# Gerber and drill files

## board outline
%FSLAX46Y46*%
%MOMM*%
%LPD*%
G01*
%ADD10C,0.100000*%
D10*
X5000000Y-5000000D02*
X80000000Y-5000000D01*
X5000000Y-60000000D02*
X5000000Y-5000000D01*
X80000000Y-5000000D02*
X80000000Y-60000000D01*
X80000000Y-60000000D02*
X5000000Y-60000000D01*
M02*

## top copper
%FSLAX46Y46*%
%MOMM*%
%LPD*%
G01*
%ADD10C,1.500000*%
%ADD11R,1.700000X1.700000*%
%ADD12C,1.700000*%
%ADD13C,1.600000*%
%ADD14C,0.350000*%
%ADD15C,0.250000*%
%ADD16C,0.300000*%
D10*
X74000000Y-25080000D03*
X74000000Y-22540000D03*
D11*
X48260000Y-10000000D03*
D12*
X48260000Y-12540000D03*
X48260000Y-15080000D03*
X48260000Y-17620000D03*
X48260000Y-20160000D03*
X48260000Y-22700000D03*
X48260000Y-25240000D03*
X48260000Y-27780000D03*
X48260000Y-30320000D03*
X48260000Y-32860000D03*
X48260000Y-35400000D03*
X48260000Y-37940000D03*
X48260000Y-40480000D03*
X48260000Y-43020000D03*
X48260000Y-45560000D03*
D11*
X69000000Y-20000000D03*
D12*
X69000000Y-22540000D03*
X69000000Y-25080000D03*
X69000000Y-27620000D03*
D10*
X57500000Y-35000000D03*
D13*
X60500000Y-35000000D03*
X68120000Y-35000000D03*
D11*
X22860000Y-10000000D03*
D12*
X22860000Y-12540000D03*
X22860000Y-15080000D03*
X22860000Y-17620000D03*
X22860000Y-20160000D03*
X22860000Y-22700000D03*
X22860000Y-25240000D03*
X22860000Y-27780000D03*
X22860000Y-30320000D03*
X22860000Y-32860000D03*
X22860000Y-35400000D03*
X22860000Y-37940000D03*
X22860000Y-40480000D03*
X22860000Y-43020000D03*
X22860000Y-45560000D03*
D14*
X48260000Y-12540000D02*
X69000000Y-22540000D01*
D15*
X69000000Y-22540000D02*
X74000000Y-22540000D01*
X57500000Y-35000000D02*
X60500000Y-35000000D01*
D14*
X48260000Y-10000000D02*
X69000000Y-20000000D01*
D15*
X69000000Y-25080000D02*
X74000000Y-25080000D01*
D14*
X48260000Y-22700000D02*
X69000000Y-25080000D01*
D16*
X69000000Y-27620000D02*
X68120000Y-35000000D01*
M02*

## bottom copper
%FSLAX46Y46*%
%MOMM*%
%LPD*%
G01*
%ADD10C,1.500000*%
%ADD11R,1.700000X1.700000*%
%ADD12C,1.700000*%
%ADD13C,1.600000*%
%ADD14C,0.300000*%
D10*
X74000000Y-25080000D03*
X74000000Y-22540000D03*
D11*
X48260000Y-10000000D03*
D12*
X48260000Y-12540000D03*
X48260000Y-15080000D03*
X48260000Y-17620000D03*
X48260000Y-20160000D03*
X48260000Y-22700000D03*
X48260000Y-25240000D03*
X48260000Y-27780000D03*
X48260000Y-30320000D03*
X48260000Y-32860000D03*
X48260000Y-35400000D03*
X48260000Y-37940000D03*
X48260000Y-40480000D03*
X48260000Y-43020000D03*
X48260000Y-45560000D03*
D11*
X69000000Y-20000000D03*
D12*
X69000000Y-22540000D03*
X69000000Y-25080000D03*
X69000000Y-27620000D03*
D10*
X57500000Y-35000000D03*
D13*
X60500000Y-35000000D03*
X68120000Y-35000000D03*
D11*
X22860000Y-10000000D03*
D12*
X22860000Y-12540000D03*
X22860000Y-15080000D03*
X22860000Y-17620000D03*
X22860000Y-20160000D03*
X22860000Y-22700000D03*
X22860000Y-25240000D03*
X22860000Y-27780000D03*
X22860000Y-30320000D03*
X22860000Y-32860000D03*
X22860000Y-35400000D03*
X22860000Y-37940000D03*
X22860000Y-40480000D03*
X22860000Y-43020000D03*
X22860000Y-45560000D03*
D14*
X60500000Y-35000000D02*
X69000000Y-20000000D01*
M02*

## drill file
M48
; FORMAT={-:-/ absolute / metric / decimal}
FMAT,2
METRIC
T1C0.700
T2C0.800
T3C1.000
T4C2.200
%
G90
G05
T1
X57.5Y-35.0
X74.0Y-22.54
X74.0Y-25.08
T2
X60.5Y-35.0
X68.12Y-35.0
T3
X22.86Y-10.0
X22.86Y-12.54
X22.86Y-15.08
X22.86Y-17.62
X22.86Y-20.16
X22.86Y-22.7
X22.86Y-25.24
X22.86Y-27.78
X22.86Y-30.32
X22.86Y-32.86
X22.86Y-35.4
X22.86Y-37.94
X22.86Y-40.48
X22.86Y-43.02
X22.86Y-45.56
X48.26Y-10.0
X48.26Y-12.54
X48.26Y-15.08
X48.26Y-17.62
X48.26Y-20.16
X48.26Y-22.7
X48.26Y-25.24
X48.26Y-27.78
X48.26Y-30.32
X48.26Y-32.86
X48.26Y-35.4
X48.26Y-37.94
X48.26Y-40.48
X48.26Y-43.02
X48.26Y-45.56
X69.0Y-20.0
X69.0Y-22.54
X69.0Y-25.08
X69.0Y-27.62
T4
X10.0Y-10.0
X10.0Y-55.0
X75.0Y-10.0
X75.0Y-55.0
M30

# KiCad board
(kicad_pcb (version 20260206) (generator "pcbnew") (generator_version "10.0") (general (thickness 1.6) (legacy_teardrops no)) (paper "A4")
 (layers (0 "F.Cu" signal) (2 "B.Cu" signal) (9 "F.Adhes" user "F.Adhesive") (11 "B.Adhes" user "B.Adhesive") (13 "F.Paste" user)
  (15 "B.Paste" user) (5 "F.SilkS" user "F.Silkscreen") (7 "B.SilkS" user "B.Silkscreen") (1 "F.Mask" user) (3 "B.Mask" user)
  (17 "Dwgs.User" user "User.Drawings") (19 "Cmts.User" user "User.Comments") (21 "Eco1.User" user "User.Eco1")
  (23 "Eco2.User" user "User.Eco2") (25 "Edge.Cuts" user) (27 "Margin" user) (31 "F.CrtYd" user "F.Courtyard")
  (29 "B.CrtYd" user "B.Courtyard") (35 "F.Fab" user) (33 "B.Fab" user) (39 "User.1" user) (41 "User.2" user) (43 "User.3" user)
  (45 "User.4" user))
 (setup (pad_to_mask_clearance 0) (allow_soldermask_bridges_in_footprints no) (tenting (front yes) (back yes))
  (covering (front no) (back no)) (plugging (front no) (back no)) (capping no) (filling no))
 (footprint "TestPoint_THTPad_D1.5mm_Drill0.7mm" (layer "F.Cu") (at 74 25.08)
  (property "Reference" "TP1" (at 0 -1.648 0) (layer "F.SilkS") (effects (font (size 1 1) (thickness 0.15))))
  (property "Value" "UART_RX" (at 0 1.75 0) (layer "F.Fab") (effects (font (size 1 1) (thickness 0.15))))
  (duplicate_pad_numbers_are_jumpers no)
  (pad "1" thru_hole circle (at 0 0) (size 1.5 1.5) (drill 0.7) (layers "*.Cu" "*.Mask") (remove_unused_layers no) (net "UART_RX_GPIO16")))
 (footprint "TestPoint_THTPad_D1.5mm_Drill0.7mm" (layer "F.Cu") (at 74 22.54)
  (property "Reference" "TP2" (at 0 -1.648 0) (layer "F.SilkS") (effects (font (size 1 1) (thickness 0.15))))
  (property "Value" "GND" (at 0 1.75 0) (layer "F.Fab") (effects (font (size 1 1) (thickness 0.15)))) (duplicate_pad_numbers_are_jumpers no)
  (pad "1" thru_hole circle (at 0 0) (size 1.5 1.5) (drill 0.7) (layers "*.Cu" "*.Mask") (remove_unused_layers no) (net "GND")))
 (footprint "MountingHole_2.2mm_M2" (layer "F.Cu") (at 10 55)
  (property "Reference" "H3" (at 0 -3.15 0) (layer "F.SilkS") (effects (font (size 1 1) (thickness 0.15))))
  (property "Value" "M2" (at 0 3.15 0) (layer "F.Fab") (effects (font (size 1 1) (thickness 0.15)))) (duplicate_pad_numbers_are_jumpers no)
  (pad "" np_thru_hole circle (at 0 0) (size 2.2 2.2) (drill 2.2) (layers "*.Cu" "*.Mask")))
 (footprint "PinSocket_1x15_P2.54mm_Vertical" (layer "F.Cu") (at 48.26 10)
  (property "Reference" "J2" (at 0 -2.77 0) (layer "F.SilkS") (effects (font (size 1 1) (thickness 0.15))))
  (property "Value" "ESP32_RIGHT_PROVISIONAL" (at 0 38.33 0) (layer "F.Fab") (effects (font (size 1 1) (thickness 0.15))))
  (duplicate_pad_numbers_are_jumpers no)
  (pad "1" thru_hole rect (at 0 0) (size 1.7 1.7) (drill 1) (layers "*.Cu" "*.Mask") (remove_unused_layers no) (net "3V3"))
  (pad "2" thru_hole circle (at 0 2.54) (size 1.7 1.7) (drill 1) (layers "*.Cu" "*.Mask") (remove_unused_layers no) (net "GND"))
  (pad "3" thru_hole circle (at 0 5.08) (size 1.7 1.7) (drill 1) (layers "*.Cu" "*.Mask") (remove_unused_layers no))
  (pad "4" thru_hole circle (at 0 7.62) (size 1.7 1.7) (drill 1) (layers "*.Cu" "*.Mask") (remove_unused_layers no))
  (pad "5" thru_hole circle (at 0 10.16) (size 1.7 1.7) (drill 1) (layers "*.Cu" "*.Mask") (remove_unused_layers no))
  (pad "6" thru_hole circle (at 0 12.7) (size 1.7 1.7) (drill 1) (layers "*.Cu" "*.Mask") (remove_unused_layers no) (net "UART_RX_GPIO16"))
  (pad "7" thru_hole circle (at 0 15.24) (size 1.7 1.7) (drill 1) (layers "*.Cu" "*.Mask") (remove_unused_layers no))
  (pad "8" thru_hole circle (at 0 17.78) (size 1.7 1.7) (drill 1) (layers "*.Cu" "*.Mask") (remove_unused_layers no))
  (pad "9" thru_hole circle (at 0 20.32) (size 1.7 1.7) (drill 1) (layers "*.Cu" "*.Mask") (remove_unused_layers no))
  (pad "10" thru_hole circle (at 0 22.86) (size 1.7 1.7) (drill 1) (layers "*.Cu" "*.Mask") (remove_unused_layers no))
  (pad "11" thru_hole circle (at 0 25.4) (size 1.7 1.7) (drill 1) (layers "*.Cu" "*.Mask") (remove_unused_layers no))
  (pad "12" thru_hole circle (at 0 27.94) (size 1.7 1.7) (drill 1) (layers "*.Cu" "*.Mask") (remove_unused_layers no))
  (pad "13" thru_hole circle (at 0 30.48) (size 1.7 1.7) (drill 1) (layers "*.Cu" "*.Mask") (remove_unused_layers no))
  (pad "14" thru_hole circle (at 0 33.02) (size 1.7 1.7) (drill 1) (layers "*.Cu" "*.Mask") (remove_unused_layers no))
  (pad "15" thru_hole circle (at 0 35.56) (size 1.7 1.7) (drill 1) (layers "*.Cu" "*.Mask") (remove_unused_layers no)))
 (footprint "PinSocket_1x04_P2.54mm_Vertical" (layer "F.Cu") (at 69 20)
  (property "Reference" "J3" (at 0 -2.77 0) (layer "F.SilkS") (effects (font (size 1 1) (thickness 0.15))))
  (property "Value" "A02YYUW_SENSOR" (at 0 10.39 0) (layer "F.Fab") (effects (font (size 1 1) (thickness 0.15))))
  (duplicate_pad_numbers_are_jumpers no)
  (pad "1" thru_hole rect (at 0 0) (size 1.7 1.7) (drill 1) (layers "*.Cu" "*.Mask") (remove_unused_layers no) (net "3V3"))
  (pad "2" thru_hole circle (at 0 2.54) (size 1.7 1.7) (drill 1) (layers "*.Cu" "*.Mask") (remove_unused_layers no) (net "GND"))
  (pad "3" thru_hole circle (at 0 5.08) (size 1.7 1.7) (drill 1) (layers "*.Cu" "*.Mask") (remove_unused_layers no) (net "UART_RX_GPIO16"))
  (pad "4" thru_hole circle (at 0 7.62) (size 1.7 1.7) (drill 1) (layers "*.Cu" "*.Mask") (remove_unused_layers no) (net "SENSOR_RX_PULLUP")))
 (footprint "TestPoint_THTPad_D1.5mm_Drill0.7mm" (layer "F.Cu") (at 57.5 35)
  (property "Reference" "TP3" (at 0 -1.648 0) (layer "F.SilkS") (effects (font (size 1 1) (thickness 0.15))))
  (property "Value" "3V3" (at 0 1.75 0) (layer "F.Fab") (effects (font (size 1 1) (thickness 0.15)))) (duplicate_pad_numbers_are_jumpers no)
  (pad "1" thru_hole circle (at 0 0) (size 1.5 1.5) (drill 0.7) (layers "*.Cu" "*.Mask") (remove_unused_layers no) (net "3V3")))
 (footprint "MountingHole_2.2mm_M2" (layer "F.Cu") (at 10 10)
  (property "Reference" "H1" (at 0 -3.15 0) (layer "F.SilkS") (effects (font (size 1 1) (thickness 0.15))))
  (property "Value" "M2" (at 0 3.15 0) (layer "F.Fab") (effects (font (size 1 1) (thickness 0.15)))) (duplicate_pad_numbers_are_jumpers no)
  (pad "" np_thru_hole circle (at 0 0) (size 2.2 2.2) (drill 2.2) (layers "*.Cu" "*.Mask")))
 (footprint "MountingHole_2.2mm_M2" (layer "F.Cu") (at 75 10)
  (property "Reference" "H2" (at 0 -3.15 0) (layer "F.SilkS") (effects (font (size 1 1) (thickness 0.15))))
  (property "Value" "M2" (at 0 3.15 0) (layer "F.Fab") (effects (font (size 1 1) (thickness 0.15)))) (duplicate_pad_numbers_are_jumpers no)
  (pad "" np_thru_hole circle (at 0 0) (size 2.2 2.2) (drill 2.2) (layers "*.Cu" "*.Mask")))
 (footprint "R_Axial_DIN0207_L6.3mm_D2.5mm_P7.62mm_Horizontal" (layer "F.Cu") (at 60.5 35)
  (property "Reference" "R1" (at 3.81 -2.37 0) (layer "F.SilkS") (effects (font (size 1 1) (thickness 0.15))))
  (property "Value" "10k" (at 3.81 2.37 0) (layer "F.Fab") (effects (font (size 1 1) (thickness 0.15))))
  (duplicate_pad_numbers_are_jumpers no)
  (pad "1" thru_hole circle (at 0 0) (size 1.6 1.6) (drill 0.8) (layers "*.Cu" "*.Mask") (remove_unused_layers no) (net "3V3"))
  (pad "2" thru_hole circle (at 7.62 0) (size 1.6 1.6) (drill 0.8) (layers "*.Cu" "*.Mask") (remove_unused_layers no)
   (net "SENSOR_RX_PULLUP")))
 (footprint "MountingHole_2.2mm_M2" (layer "F.Cu") (at 75 55)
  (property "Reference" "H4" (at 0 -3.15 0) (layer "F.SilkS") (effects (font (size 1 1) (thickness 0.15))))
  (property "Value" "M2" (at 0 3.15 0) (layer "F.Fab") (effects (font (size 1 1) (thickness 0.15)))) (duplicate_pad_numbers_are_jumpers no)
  (pad "" np_thru_hole circle (at 0 0) (size 2.2 2.2) (drill 2.2) (layers "*.Cu" "*.Mask")))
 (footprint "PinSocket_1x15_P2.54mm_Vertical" (layer "F.Cu") (at 22.86 10)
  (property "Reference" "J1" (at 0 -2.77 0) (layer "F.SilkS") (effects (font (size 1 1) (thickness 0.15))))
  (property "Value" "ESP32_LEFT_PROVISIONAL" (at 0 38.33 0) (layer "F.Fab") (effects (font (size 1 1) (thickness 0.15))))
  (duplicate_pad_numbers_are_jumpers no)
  (pad "1" thru_hole rect (at 0 0) (size 1.7 1.7) (drill 1) (layers "*.Cu" "*.Mask") (remove_unused_layers no))
  (pad "2" thru_hole circle (at 0 2.54) (size 1.7 1.7) (drill 1) (layers "*.Cu" "*.Mask") (remove_unused_layers no))
  (pad "3" thru_hole circle (at 0 5.08) (size 1.7 1.7) (drill 1) (layers "*.Cu" "*.Mask") (remove_unused_layers no))
  (pad "4" thru_hole circle (at 0 7.62) (size 1.7 1.7) (drill 1) (layers "*.Cu" "*.Mask") (remove_unused_layers no))
  (pad "5" thru_hole circle (at 0 10.16) (size 1.7 1.7) (drill 1) (layers "*.Cu" "*.Mask") (remove_unused_layers no))
  (pad "6" thru_hole circle (at 0 12.7) (size 1.7 1.7) (drill 1) (layers "*.Cu" "*.Mask") (remove_unused_layers no))
  (pad "7" thru_hole circle (at 0 15.24) (size 1.7 1.7) (drill 1) (layers "*.Cu" "*.Mask") (remove_unused_layers no))
  (pad "8" thru_hole circle (at 0 17.78) (size 1.7 1.7) (drill 1) (layers "*.Cu" "*.Mask") (remove_unused_layers no))
  (pad "9" thru_hole circle (at 0 20.32) (size 1.7 1.7) (drill 1) (layers "*.Cu" "*.Mask") (remove_unused_layers no))
  (pad "10" thru_hole circle (at 0 22.86) (size 1.7 1.7) (drill 1) (layers "*.Cu" "*.Mask") (remove_unused_layers no))
  (pad "11" thru_hole circle (at 0 25.4) (size 1.7 1.7) (drill 1) (layers "*.Cu" "*.Mask") (remove_unused_layers no))
  (pad "12" thru_hole circle (at 0 27.94) (size 1.7 1.7) (drill 1) (layers "*.Cu" "*.Mask") (remove_unused_layers no))
  (pad "13" thru_hole circle (at 0 30.48) (size 1.7 1.7) (drill 1) (layers "*.Cu" "*.Mask") (remove_unused_layers no))
  (pad "14" thru_hole circle (at 0 33.02) (size 1.7 1.7) (drill 1) (layers "*.Cu" "*.Mask") (remove_unused_layers no))
  (pad "15" thru_hole circle (at 0 35.56) (size 1.7 1.7) (drill 1) (layers "*.Cu" "*.Mask") (remove_unused_layers no)))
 (gr_line (start 5 5) (end 80 5) (stroke (width 0.1) (type default)) (layer "Edge.Cuts"))
 (gr_line (start 5 60) (end 5 5) (stroke (width 0.1) (type default)) (layer "Edge.Cuts"))
 (gr_line (start 80 5) (end 80 60) (stroke (width 0.1) (type default)) (layer "Edge.Cuts"))
 (gr_line (start 80 60) (end 5 60) (stroke (width 0.1) (type default)) (layer "Edge.Cuts"))
 (segment (start 48.26 12.54) (end 69 22.54) (width 0.35) (layer "F.Cu") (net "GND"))
 (segment (start 69 22.54) (end 74 22.54) (width 0.25) (layer "F.Cu") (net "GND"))
 (segment (start 57.5 35) (end 60.5 35) (width 0.25) (layer "F.Cu") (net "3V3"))
 (segment (start 48.26 10) (end 69 20) (width 0.35) (layer "F.Cu") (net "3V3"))
 (segment (start 60.5 35) (end 69 20) (width 0.3) (layer "B.Cu") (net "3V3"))
 (segment (start 69 25.08) (end 74 25.08) (width 0.25) (layer "F.Cu") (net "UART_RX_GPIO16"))
 (segment (start 48.26 22.7) (end 69 25.08) (width 0.35) (layer "F.Cu") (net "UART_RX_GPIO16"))
 (segment (start 69 27.62) (end 68.12 35) (width 0.3) (layer "F.Cu") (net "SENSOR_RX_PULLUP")))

